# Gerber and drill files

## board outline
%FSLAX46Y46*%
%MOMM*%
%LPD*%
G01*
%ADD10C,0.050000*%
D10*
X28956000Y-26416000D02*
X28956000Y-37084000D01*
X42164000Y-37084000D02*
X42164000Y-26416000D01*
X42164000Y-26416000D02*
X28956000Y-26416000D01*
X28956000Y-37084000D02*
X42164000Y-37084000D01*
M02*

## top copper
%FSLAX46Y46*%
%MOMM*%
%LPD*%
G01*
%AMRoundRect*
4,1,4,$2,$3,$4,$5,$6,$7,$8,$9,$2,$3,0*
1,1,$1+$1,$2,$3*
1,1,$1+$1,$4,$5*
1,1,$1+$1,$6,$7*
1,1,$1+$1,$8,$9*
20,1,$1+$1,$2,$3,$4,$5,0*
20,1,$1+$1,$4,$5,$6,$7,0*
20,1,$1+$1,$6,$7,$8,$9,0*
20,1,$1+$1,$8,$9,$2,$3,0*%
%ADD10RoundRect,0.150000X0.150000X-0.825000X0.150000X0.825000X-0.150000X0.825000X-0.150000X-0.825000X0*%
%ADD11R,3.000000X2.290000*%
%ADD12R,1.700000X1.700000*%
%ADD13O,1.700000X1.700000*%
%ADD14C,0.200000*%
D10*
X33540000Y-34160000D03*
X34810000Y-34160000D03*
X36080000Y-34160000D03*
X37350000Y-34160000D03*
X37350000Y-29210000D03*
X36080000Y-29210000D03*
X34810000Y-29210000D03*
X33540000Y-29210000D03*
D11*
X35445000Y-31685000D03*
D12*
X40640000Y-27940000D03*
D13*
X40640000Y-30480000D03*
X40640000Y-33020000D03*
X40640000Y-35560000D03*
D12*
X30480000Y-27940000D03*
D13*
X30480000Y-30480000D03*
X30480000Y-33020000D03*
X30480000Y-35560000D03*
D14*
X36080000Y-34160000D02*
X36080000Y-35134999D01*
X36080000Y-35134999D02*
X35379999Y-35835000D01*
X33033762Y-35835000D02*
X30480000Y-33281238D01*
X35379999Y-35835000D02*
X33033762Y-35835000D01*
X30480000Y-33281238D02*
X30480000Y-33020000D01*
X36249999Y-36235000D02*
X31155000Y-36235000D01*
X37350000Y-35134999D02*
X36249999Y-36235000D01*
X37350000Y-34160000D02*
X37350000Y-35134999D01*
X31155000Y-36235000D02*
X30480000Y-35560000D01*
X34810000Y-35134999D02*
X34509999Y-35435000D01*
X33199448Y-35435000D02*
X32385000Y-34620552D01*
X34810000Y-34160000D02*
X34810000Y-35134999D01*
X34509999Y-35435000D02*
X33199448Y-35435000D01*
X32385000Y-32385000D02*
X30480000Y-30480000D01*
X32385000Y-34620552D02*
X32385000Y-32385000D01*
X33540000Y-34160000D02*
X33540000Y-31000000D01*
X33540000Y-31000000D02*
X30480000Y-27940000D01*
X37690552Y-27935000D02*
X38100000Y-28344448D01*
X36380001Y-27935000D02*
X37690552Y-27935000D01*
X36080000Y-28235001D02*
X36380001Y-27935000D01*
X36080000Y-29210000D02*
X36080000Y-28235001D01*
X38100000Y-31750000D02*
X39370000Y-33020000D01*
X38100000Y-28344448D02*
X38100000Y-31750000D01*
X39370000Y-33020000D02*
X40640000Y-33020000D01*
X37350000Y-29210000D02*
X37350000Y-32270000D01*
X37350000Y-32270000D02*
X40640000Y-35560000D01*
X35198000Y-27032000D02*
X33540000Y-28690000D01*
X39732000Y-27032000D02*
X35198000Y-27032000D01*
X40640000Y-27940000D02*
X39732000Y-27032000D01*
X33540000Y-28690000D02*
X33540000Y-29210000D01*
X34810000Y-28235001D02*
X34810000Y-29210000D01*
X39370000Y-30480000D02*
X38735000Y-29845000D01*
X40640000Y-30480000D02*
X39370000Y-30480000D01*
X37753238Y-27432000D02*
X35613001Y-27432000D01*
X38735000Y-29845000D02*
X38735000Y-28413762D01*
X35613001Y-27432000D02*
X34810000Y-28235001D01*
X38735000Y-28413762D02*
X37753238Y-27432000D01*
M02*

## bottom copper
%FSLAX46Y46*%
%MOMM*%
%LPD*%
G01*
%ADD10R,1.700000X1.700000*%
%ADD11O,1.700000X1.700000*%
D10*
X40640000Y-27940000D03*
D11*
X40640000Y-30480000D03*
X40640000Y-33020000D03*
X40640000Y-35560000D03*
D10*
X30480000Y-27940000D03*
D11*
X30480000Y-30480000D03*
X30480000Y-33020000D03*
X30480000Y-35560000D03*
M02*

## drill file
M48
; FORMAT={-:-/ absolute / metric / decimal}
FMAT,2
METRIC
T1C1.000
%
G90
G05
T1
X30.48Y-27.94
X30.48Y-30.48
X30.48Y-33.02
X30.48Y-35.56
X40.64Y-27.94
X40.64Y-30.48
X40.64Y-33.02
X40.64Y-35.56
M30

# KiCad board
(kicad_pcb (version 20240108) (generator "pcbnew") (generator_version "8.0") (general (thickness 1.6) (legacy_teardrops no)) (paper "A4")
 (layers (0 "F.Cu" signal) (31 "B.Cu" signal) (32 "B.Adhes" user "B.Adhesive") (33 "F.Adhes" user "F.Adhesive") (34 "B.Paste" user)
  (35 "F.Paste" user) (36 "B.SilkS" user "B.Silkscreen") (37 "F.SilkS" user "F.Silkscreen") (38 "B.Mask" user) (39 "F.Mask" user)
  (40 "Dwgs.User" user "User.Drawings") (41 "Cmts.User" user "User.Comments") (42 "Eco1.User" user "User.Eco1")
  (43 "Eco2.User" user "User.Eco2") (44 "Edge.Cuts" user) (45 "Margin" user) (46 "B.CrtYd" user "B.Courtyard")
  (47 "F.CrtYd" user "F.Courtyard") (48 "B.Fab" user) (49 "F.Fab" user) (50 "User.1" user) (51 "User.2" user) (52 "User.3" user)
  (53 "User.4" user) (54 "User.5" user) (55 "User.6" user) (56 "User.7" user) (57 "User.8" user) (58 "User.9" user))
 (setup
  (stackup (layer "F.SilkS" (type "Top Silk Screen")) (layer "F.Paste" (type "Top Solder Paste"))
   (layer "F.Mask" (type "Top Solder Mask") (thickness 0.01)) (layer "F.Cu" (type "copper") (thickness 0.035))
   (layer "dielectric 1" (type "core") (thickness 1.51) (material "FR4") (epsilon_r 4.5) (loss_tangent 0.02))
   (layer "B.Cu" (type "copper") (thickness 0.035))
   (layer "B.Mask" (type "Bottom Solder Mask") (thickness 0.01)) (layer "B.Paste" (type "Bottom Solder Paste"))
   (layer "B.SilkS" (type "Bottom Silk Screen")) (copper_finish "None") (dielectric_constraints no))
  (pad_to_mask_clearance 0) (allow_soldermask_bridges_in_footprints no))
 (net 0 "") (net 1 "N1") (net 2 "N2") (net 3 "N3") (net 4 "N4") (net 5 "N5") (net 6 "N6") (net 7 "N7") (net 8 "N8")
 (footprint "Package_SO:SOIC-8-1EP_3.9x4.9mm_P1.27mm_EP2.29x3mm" (layer "F.Cu") (at 35.445 31.685 90)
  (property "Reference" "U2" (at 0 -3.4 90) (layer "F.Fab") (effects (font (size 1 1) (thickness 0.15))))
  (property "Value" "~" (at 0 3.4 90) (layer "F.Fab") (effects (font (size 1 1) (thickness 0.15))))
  (pad "" smd roundrect (at -0.57 -0.75 90) (size 0.92 1.21) (layers "F.Paste") (roundrect_rratio 0.25))
  (pad "" smd roundrect (at -0.57 0.75 90) (size 0.92 1.21) (layers "F.Paste") (roundrect_rratio 0.25))
  (pad "" smd roundrect (at 0.57 -0.75 90) (size 0.92 1.21) (layers "F.Paste") (roundrect_rratio 0.25))
  (pad "" smd roundrect (at 0.57 0.75 90) (size 0.92 1.21) (layers "F.Paste") (roundrect_rratio 0.25))
  (pad "1" smd roundrect (at -2.475 -1.905 90) (size 1.95 0.6) (layers "F.Cu" "F.Paste" "F.Mask") (roundrect_rratio 0.25) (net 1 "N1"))
  (pad "2" smd roundrect (at -2.475 -0.635 90) (size 1.95 0.6) (layers "F.Cu" "F.Paste" "F.Mask") (roundrect_rratio 0.25) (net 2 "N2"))
  (pad "3" smd roundrect (at -2.475 0.635 90) (size 1.95 0.6) (layers "F.Cu" "F.Paste" "F.Mask") (roundrect_rratio 0.25) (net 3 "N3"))
  (pad "4" smd roundrect (at -2.475 1.905 90) (size 1.95 0.6) (layers "F.Cu" "F.Paste" "F.Mask") (roundrect_rratio 0.25) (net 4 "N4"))
  (pad "5" smd roundrect (at 2.475 1.905 90) (size 1.95 0.6) (layers "F.Cu" "F.Paste" "F.Mask") (roundrect_rratio 0.25) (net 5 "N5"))
  (pad "6" smd roundrect (at 2.475 0.635 90) (size 1.95 0.6) (layers "F.Cu" "F.Paste" "F.Mask") (roundrect_rratio 0.25) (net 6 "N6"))
  (pad "7" smd roundrect (at 2.475 -0.635 90) (size 1.95 0.6) (layers "F.Cu" "F.Paste" "F.Mask") (roundrect_rratio 0.25) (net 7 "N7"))
  (pad "8" smd roundrect (at 2.475 -1.905 90) (size 1.95 0.6) (layers "F.Cu" "F.Paste" "F.Mask") (roundrect_rratio 0.25) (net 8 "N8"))
  (pad "9" smd rect (at 0 0 90) (size 2.29 3) (layers "F.Cu" "F.Mask") (zone_connect 2)))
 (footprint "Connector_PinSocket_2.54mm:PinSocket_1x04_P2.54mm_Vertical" (layer "B.Cu") (at 40.64 27.94 180)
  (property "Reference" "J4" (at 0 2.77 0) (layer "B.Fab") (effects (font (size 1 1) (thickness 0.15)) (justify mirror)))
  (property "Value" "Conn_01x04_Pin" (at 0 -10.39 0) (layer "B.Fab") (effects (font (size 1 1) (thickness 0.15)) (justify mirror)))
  (pad "1" thru_hole rect (at 0 0 180) (size 1.7 1.7) (drill 1) (layers "*.Cu" "*.Mask") (remove_unused_layers no) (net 8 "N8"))
  (pad "2" thru_hole oval (at 0 -2.54 180) (size 1.7 1.7) (drill 1) (layers "*.Cu" "*.Mask") (remove_unused_layers no) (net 7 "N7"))
  (pad "3" thru_hole oval (at 0 -5.08 180) (size 1.7 1.7) (drill 1) (layers "*.Cu" "*.Mask") (remove_unused_layers no) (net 6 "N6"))
  (pad "4" thru_hole oval (at 0 -7.62 180) (size 1.7 1.7) (drill 1) (layers "*.Cu" "*.Mask") (remove_unused_layers no) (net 5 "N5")))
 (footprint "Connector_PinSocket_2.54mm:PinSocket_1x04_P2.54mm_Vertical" (layer "B.Cu") (at 30.48 27.94 180)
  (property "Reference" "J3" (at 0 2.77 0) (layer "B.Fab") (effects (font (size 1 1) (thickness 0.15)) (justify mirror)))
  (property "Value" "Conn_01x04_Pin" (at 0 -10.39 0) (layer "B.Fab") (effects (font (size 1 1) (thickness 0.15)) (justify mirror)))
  (pad "1" thru_hole rect (at 0 0 180) (size 1.7 1.7) (drill 1) (layers "*.Cu" "*.Mask") (remove_unused_layers no) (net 1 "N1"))
  (pad "2" thru_hole oval (at 0 -2.54 180) (size 1.7 1.7) (drill 1) (layers "*.Cu" "*.Mask") (remove_unused_layers no) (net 2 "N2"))
  (pad "3" thru_hole oval (at 0 -5.08 180) (size 1.7 1.7) (drill 1) (layers "*.Cu" "*.Mask") (remove_unused_layers no) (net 3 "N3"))
  (pad "4" thru_hole oval (at 0 -7.62 180) (size 1.7 1.7) (drill 1) (layers "*.Cu" "*.Mask") (remove_unused_layers no) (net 4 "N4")))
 (gr_line (start 28.956 26.416) (end 28.956 37.084) (stroke (width 0.05) (type default)) (layer "Edge.Cuts"))
 (gr_line (start 42.164 37.084) (end 42.164 26.416) (stroke (width 0.05) (type default)) (layer "Edge.Cuts"))
 (gr_line (start 42.164 26.416) (end 28.956 26.416) (stroke (width 0.05) (type default)) (layer "Edge.Cuts"))
 (gr_line (start 28.956 37.084) (end 42.164 37.084) (stroke (width 0.05) (type default)) (layer "Edge.Cuts"))
 (segment (start 36.08 34.16) (end 36.08 35.134999) (width 0.2) (layer "F.Cu") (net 3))
 (segment (start 36.08 35.134999) (end 35.379999 35.835) (width 0.2) (layer "F.Cu") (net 3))
 (segment (start 33.033762 35.835) (end 30.48 33.281238) (width 0.2) (layer "F.Cu") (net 3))
 (segment (start 35.379999 35.835) (end 33.033762 35.835) (width 0.2) (layer "F.Cu") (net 3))
 (segment (start 30.48 33.281238) (end 30.48 33.02) (width 0.2) (layer "F.Cu") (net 3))
 (segment (start 36.249999 36.235) (end 31.155 36.235) (width 0.2) (layer "F.Cu") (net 4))
 (segment (start 37.35 35.134999) (end 36.249999 36.235) (width 0.2) (layer "F.Cu") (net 4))
 (segment (start 37.35 34.16) (end 37.35 35.134999) (width 0.2) (layer "F.Cu") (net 4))
 (segment (start 31.155 36.235) (end 30.48 35.56) (width 0.2) (layer "F.Cu") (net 4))
 (segment (start 34.81 35.134999) (end 34.509999 35.435) (width 0.2) (layer "F.Cu") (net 2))
 (segment (start 33.199448 35.435) (end 32.385 34.620552) (width 0.2) (layer "F.Cu") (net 2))
 (segment (start 34.81 34.16) (end 34.81 35.134999) (width 0.2) (layer "F.Cu") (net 2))
 (segment (start 34.509999 35.435) (end 33.199448 35.435) (width 0.2) (layer "F.Cu") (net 2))
 (segment (start 32.385 32.385) (end 30.48 30.48) (width 0.2) (layer "F.Cu") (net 2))
 (segment (start 32.385 34.620552) (end 32.385 32.385) (width 0.2) (layer "F.Cu") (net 2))
 (segment (start 33.54 34.16) (end 33.54 31) (width 0.2) (layer "F.Cu") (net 1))
 (segment (start 33.54 31) (end 30.48 27.94) (width 0.2) (layer "F.Cu") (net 1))
 (segment (start 37.690552 27.935) (end 38.1 28.344448) (width 0.2) (layer "F.Cu") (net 6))
 (segment (start 36.380001 27.935) (end 37.690552 27.935) (width 0.2) (layer "F.Cu") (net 6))
 (segment (start 36.08 28.235001) (end 36.380001 27.935) (width 0.2) (layer "F.Cu") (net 6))
 (segment (start 36.08 29.21) (end 36.08 28.235001) (width 0.2) (layer "F.Cu") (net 6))
 (segment (start 38.1 31.75) (end 39.37 33.02) (width 0.2) (layer "F.Cu") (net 6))
 (segment (start 38.1 28.344448) (end 38.1 31.75) (width 0.2) (layer "F.Cu") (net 6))
 (segment (start 39.37 33.02) (end 40.64 33.02) (width 0.2) (layer "F.Cu") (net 6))
 (segment (start 37.35 29.21) (end 37.35 32.27) (width 0.2) (layer "F.Cu") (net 5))
 (segment (start 37.35 32.27) (end 40.64 35.56) (width 0.2) (layer "F.Cu") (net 5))
 (segment (start 35.198 27.032) (end 33.54 28.69) (width 0.2) (layer "F.Cu") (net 8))
 (segment (start 39.732 27.032) (end 35.198 27.032) (width 0.2) (layer "F.Cu") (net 8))
 (segment (start 40.64 27.94) (end 39.732 27.032) (width 0.2) (layer "F.Cu") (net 8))
 (segment (start 33.54 28.69) (end 33.54 29.21) (width 0.2) (layer "F.Cu") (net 8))
 (segment (start 34.81 28.235001) (end 34.81 29.21) (width 0.2) (layer "F.Cu") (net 7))
 (segment (start 39.37 30.48) (end 38.735 29.845) (width 0.2) (layer "F.Cu") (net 7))
 (segment (start 40.64 30.48) (end 39.37 30.48) (width 0.2) (layer "F.Cu") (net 7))
 (segment (start 37.753238 27.432) (end 35.613001 27.432) (width 0.2) (layer "F.Cu") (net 7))
 (segment (start 38.735 29.845) (end 38.735 28.413762) (width 0.2) (layer "F.Cu") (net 7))
 (segment (start 35.613001 27.432) (end 34.81 28.235001) (width 0.2) (layer "F.Cu") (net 7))
 (segment (start 38.735 28.413762) (end 37.753238 27.432) (width 0.2) (layer "F.Cu") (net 7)))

